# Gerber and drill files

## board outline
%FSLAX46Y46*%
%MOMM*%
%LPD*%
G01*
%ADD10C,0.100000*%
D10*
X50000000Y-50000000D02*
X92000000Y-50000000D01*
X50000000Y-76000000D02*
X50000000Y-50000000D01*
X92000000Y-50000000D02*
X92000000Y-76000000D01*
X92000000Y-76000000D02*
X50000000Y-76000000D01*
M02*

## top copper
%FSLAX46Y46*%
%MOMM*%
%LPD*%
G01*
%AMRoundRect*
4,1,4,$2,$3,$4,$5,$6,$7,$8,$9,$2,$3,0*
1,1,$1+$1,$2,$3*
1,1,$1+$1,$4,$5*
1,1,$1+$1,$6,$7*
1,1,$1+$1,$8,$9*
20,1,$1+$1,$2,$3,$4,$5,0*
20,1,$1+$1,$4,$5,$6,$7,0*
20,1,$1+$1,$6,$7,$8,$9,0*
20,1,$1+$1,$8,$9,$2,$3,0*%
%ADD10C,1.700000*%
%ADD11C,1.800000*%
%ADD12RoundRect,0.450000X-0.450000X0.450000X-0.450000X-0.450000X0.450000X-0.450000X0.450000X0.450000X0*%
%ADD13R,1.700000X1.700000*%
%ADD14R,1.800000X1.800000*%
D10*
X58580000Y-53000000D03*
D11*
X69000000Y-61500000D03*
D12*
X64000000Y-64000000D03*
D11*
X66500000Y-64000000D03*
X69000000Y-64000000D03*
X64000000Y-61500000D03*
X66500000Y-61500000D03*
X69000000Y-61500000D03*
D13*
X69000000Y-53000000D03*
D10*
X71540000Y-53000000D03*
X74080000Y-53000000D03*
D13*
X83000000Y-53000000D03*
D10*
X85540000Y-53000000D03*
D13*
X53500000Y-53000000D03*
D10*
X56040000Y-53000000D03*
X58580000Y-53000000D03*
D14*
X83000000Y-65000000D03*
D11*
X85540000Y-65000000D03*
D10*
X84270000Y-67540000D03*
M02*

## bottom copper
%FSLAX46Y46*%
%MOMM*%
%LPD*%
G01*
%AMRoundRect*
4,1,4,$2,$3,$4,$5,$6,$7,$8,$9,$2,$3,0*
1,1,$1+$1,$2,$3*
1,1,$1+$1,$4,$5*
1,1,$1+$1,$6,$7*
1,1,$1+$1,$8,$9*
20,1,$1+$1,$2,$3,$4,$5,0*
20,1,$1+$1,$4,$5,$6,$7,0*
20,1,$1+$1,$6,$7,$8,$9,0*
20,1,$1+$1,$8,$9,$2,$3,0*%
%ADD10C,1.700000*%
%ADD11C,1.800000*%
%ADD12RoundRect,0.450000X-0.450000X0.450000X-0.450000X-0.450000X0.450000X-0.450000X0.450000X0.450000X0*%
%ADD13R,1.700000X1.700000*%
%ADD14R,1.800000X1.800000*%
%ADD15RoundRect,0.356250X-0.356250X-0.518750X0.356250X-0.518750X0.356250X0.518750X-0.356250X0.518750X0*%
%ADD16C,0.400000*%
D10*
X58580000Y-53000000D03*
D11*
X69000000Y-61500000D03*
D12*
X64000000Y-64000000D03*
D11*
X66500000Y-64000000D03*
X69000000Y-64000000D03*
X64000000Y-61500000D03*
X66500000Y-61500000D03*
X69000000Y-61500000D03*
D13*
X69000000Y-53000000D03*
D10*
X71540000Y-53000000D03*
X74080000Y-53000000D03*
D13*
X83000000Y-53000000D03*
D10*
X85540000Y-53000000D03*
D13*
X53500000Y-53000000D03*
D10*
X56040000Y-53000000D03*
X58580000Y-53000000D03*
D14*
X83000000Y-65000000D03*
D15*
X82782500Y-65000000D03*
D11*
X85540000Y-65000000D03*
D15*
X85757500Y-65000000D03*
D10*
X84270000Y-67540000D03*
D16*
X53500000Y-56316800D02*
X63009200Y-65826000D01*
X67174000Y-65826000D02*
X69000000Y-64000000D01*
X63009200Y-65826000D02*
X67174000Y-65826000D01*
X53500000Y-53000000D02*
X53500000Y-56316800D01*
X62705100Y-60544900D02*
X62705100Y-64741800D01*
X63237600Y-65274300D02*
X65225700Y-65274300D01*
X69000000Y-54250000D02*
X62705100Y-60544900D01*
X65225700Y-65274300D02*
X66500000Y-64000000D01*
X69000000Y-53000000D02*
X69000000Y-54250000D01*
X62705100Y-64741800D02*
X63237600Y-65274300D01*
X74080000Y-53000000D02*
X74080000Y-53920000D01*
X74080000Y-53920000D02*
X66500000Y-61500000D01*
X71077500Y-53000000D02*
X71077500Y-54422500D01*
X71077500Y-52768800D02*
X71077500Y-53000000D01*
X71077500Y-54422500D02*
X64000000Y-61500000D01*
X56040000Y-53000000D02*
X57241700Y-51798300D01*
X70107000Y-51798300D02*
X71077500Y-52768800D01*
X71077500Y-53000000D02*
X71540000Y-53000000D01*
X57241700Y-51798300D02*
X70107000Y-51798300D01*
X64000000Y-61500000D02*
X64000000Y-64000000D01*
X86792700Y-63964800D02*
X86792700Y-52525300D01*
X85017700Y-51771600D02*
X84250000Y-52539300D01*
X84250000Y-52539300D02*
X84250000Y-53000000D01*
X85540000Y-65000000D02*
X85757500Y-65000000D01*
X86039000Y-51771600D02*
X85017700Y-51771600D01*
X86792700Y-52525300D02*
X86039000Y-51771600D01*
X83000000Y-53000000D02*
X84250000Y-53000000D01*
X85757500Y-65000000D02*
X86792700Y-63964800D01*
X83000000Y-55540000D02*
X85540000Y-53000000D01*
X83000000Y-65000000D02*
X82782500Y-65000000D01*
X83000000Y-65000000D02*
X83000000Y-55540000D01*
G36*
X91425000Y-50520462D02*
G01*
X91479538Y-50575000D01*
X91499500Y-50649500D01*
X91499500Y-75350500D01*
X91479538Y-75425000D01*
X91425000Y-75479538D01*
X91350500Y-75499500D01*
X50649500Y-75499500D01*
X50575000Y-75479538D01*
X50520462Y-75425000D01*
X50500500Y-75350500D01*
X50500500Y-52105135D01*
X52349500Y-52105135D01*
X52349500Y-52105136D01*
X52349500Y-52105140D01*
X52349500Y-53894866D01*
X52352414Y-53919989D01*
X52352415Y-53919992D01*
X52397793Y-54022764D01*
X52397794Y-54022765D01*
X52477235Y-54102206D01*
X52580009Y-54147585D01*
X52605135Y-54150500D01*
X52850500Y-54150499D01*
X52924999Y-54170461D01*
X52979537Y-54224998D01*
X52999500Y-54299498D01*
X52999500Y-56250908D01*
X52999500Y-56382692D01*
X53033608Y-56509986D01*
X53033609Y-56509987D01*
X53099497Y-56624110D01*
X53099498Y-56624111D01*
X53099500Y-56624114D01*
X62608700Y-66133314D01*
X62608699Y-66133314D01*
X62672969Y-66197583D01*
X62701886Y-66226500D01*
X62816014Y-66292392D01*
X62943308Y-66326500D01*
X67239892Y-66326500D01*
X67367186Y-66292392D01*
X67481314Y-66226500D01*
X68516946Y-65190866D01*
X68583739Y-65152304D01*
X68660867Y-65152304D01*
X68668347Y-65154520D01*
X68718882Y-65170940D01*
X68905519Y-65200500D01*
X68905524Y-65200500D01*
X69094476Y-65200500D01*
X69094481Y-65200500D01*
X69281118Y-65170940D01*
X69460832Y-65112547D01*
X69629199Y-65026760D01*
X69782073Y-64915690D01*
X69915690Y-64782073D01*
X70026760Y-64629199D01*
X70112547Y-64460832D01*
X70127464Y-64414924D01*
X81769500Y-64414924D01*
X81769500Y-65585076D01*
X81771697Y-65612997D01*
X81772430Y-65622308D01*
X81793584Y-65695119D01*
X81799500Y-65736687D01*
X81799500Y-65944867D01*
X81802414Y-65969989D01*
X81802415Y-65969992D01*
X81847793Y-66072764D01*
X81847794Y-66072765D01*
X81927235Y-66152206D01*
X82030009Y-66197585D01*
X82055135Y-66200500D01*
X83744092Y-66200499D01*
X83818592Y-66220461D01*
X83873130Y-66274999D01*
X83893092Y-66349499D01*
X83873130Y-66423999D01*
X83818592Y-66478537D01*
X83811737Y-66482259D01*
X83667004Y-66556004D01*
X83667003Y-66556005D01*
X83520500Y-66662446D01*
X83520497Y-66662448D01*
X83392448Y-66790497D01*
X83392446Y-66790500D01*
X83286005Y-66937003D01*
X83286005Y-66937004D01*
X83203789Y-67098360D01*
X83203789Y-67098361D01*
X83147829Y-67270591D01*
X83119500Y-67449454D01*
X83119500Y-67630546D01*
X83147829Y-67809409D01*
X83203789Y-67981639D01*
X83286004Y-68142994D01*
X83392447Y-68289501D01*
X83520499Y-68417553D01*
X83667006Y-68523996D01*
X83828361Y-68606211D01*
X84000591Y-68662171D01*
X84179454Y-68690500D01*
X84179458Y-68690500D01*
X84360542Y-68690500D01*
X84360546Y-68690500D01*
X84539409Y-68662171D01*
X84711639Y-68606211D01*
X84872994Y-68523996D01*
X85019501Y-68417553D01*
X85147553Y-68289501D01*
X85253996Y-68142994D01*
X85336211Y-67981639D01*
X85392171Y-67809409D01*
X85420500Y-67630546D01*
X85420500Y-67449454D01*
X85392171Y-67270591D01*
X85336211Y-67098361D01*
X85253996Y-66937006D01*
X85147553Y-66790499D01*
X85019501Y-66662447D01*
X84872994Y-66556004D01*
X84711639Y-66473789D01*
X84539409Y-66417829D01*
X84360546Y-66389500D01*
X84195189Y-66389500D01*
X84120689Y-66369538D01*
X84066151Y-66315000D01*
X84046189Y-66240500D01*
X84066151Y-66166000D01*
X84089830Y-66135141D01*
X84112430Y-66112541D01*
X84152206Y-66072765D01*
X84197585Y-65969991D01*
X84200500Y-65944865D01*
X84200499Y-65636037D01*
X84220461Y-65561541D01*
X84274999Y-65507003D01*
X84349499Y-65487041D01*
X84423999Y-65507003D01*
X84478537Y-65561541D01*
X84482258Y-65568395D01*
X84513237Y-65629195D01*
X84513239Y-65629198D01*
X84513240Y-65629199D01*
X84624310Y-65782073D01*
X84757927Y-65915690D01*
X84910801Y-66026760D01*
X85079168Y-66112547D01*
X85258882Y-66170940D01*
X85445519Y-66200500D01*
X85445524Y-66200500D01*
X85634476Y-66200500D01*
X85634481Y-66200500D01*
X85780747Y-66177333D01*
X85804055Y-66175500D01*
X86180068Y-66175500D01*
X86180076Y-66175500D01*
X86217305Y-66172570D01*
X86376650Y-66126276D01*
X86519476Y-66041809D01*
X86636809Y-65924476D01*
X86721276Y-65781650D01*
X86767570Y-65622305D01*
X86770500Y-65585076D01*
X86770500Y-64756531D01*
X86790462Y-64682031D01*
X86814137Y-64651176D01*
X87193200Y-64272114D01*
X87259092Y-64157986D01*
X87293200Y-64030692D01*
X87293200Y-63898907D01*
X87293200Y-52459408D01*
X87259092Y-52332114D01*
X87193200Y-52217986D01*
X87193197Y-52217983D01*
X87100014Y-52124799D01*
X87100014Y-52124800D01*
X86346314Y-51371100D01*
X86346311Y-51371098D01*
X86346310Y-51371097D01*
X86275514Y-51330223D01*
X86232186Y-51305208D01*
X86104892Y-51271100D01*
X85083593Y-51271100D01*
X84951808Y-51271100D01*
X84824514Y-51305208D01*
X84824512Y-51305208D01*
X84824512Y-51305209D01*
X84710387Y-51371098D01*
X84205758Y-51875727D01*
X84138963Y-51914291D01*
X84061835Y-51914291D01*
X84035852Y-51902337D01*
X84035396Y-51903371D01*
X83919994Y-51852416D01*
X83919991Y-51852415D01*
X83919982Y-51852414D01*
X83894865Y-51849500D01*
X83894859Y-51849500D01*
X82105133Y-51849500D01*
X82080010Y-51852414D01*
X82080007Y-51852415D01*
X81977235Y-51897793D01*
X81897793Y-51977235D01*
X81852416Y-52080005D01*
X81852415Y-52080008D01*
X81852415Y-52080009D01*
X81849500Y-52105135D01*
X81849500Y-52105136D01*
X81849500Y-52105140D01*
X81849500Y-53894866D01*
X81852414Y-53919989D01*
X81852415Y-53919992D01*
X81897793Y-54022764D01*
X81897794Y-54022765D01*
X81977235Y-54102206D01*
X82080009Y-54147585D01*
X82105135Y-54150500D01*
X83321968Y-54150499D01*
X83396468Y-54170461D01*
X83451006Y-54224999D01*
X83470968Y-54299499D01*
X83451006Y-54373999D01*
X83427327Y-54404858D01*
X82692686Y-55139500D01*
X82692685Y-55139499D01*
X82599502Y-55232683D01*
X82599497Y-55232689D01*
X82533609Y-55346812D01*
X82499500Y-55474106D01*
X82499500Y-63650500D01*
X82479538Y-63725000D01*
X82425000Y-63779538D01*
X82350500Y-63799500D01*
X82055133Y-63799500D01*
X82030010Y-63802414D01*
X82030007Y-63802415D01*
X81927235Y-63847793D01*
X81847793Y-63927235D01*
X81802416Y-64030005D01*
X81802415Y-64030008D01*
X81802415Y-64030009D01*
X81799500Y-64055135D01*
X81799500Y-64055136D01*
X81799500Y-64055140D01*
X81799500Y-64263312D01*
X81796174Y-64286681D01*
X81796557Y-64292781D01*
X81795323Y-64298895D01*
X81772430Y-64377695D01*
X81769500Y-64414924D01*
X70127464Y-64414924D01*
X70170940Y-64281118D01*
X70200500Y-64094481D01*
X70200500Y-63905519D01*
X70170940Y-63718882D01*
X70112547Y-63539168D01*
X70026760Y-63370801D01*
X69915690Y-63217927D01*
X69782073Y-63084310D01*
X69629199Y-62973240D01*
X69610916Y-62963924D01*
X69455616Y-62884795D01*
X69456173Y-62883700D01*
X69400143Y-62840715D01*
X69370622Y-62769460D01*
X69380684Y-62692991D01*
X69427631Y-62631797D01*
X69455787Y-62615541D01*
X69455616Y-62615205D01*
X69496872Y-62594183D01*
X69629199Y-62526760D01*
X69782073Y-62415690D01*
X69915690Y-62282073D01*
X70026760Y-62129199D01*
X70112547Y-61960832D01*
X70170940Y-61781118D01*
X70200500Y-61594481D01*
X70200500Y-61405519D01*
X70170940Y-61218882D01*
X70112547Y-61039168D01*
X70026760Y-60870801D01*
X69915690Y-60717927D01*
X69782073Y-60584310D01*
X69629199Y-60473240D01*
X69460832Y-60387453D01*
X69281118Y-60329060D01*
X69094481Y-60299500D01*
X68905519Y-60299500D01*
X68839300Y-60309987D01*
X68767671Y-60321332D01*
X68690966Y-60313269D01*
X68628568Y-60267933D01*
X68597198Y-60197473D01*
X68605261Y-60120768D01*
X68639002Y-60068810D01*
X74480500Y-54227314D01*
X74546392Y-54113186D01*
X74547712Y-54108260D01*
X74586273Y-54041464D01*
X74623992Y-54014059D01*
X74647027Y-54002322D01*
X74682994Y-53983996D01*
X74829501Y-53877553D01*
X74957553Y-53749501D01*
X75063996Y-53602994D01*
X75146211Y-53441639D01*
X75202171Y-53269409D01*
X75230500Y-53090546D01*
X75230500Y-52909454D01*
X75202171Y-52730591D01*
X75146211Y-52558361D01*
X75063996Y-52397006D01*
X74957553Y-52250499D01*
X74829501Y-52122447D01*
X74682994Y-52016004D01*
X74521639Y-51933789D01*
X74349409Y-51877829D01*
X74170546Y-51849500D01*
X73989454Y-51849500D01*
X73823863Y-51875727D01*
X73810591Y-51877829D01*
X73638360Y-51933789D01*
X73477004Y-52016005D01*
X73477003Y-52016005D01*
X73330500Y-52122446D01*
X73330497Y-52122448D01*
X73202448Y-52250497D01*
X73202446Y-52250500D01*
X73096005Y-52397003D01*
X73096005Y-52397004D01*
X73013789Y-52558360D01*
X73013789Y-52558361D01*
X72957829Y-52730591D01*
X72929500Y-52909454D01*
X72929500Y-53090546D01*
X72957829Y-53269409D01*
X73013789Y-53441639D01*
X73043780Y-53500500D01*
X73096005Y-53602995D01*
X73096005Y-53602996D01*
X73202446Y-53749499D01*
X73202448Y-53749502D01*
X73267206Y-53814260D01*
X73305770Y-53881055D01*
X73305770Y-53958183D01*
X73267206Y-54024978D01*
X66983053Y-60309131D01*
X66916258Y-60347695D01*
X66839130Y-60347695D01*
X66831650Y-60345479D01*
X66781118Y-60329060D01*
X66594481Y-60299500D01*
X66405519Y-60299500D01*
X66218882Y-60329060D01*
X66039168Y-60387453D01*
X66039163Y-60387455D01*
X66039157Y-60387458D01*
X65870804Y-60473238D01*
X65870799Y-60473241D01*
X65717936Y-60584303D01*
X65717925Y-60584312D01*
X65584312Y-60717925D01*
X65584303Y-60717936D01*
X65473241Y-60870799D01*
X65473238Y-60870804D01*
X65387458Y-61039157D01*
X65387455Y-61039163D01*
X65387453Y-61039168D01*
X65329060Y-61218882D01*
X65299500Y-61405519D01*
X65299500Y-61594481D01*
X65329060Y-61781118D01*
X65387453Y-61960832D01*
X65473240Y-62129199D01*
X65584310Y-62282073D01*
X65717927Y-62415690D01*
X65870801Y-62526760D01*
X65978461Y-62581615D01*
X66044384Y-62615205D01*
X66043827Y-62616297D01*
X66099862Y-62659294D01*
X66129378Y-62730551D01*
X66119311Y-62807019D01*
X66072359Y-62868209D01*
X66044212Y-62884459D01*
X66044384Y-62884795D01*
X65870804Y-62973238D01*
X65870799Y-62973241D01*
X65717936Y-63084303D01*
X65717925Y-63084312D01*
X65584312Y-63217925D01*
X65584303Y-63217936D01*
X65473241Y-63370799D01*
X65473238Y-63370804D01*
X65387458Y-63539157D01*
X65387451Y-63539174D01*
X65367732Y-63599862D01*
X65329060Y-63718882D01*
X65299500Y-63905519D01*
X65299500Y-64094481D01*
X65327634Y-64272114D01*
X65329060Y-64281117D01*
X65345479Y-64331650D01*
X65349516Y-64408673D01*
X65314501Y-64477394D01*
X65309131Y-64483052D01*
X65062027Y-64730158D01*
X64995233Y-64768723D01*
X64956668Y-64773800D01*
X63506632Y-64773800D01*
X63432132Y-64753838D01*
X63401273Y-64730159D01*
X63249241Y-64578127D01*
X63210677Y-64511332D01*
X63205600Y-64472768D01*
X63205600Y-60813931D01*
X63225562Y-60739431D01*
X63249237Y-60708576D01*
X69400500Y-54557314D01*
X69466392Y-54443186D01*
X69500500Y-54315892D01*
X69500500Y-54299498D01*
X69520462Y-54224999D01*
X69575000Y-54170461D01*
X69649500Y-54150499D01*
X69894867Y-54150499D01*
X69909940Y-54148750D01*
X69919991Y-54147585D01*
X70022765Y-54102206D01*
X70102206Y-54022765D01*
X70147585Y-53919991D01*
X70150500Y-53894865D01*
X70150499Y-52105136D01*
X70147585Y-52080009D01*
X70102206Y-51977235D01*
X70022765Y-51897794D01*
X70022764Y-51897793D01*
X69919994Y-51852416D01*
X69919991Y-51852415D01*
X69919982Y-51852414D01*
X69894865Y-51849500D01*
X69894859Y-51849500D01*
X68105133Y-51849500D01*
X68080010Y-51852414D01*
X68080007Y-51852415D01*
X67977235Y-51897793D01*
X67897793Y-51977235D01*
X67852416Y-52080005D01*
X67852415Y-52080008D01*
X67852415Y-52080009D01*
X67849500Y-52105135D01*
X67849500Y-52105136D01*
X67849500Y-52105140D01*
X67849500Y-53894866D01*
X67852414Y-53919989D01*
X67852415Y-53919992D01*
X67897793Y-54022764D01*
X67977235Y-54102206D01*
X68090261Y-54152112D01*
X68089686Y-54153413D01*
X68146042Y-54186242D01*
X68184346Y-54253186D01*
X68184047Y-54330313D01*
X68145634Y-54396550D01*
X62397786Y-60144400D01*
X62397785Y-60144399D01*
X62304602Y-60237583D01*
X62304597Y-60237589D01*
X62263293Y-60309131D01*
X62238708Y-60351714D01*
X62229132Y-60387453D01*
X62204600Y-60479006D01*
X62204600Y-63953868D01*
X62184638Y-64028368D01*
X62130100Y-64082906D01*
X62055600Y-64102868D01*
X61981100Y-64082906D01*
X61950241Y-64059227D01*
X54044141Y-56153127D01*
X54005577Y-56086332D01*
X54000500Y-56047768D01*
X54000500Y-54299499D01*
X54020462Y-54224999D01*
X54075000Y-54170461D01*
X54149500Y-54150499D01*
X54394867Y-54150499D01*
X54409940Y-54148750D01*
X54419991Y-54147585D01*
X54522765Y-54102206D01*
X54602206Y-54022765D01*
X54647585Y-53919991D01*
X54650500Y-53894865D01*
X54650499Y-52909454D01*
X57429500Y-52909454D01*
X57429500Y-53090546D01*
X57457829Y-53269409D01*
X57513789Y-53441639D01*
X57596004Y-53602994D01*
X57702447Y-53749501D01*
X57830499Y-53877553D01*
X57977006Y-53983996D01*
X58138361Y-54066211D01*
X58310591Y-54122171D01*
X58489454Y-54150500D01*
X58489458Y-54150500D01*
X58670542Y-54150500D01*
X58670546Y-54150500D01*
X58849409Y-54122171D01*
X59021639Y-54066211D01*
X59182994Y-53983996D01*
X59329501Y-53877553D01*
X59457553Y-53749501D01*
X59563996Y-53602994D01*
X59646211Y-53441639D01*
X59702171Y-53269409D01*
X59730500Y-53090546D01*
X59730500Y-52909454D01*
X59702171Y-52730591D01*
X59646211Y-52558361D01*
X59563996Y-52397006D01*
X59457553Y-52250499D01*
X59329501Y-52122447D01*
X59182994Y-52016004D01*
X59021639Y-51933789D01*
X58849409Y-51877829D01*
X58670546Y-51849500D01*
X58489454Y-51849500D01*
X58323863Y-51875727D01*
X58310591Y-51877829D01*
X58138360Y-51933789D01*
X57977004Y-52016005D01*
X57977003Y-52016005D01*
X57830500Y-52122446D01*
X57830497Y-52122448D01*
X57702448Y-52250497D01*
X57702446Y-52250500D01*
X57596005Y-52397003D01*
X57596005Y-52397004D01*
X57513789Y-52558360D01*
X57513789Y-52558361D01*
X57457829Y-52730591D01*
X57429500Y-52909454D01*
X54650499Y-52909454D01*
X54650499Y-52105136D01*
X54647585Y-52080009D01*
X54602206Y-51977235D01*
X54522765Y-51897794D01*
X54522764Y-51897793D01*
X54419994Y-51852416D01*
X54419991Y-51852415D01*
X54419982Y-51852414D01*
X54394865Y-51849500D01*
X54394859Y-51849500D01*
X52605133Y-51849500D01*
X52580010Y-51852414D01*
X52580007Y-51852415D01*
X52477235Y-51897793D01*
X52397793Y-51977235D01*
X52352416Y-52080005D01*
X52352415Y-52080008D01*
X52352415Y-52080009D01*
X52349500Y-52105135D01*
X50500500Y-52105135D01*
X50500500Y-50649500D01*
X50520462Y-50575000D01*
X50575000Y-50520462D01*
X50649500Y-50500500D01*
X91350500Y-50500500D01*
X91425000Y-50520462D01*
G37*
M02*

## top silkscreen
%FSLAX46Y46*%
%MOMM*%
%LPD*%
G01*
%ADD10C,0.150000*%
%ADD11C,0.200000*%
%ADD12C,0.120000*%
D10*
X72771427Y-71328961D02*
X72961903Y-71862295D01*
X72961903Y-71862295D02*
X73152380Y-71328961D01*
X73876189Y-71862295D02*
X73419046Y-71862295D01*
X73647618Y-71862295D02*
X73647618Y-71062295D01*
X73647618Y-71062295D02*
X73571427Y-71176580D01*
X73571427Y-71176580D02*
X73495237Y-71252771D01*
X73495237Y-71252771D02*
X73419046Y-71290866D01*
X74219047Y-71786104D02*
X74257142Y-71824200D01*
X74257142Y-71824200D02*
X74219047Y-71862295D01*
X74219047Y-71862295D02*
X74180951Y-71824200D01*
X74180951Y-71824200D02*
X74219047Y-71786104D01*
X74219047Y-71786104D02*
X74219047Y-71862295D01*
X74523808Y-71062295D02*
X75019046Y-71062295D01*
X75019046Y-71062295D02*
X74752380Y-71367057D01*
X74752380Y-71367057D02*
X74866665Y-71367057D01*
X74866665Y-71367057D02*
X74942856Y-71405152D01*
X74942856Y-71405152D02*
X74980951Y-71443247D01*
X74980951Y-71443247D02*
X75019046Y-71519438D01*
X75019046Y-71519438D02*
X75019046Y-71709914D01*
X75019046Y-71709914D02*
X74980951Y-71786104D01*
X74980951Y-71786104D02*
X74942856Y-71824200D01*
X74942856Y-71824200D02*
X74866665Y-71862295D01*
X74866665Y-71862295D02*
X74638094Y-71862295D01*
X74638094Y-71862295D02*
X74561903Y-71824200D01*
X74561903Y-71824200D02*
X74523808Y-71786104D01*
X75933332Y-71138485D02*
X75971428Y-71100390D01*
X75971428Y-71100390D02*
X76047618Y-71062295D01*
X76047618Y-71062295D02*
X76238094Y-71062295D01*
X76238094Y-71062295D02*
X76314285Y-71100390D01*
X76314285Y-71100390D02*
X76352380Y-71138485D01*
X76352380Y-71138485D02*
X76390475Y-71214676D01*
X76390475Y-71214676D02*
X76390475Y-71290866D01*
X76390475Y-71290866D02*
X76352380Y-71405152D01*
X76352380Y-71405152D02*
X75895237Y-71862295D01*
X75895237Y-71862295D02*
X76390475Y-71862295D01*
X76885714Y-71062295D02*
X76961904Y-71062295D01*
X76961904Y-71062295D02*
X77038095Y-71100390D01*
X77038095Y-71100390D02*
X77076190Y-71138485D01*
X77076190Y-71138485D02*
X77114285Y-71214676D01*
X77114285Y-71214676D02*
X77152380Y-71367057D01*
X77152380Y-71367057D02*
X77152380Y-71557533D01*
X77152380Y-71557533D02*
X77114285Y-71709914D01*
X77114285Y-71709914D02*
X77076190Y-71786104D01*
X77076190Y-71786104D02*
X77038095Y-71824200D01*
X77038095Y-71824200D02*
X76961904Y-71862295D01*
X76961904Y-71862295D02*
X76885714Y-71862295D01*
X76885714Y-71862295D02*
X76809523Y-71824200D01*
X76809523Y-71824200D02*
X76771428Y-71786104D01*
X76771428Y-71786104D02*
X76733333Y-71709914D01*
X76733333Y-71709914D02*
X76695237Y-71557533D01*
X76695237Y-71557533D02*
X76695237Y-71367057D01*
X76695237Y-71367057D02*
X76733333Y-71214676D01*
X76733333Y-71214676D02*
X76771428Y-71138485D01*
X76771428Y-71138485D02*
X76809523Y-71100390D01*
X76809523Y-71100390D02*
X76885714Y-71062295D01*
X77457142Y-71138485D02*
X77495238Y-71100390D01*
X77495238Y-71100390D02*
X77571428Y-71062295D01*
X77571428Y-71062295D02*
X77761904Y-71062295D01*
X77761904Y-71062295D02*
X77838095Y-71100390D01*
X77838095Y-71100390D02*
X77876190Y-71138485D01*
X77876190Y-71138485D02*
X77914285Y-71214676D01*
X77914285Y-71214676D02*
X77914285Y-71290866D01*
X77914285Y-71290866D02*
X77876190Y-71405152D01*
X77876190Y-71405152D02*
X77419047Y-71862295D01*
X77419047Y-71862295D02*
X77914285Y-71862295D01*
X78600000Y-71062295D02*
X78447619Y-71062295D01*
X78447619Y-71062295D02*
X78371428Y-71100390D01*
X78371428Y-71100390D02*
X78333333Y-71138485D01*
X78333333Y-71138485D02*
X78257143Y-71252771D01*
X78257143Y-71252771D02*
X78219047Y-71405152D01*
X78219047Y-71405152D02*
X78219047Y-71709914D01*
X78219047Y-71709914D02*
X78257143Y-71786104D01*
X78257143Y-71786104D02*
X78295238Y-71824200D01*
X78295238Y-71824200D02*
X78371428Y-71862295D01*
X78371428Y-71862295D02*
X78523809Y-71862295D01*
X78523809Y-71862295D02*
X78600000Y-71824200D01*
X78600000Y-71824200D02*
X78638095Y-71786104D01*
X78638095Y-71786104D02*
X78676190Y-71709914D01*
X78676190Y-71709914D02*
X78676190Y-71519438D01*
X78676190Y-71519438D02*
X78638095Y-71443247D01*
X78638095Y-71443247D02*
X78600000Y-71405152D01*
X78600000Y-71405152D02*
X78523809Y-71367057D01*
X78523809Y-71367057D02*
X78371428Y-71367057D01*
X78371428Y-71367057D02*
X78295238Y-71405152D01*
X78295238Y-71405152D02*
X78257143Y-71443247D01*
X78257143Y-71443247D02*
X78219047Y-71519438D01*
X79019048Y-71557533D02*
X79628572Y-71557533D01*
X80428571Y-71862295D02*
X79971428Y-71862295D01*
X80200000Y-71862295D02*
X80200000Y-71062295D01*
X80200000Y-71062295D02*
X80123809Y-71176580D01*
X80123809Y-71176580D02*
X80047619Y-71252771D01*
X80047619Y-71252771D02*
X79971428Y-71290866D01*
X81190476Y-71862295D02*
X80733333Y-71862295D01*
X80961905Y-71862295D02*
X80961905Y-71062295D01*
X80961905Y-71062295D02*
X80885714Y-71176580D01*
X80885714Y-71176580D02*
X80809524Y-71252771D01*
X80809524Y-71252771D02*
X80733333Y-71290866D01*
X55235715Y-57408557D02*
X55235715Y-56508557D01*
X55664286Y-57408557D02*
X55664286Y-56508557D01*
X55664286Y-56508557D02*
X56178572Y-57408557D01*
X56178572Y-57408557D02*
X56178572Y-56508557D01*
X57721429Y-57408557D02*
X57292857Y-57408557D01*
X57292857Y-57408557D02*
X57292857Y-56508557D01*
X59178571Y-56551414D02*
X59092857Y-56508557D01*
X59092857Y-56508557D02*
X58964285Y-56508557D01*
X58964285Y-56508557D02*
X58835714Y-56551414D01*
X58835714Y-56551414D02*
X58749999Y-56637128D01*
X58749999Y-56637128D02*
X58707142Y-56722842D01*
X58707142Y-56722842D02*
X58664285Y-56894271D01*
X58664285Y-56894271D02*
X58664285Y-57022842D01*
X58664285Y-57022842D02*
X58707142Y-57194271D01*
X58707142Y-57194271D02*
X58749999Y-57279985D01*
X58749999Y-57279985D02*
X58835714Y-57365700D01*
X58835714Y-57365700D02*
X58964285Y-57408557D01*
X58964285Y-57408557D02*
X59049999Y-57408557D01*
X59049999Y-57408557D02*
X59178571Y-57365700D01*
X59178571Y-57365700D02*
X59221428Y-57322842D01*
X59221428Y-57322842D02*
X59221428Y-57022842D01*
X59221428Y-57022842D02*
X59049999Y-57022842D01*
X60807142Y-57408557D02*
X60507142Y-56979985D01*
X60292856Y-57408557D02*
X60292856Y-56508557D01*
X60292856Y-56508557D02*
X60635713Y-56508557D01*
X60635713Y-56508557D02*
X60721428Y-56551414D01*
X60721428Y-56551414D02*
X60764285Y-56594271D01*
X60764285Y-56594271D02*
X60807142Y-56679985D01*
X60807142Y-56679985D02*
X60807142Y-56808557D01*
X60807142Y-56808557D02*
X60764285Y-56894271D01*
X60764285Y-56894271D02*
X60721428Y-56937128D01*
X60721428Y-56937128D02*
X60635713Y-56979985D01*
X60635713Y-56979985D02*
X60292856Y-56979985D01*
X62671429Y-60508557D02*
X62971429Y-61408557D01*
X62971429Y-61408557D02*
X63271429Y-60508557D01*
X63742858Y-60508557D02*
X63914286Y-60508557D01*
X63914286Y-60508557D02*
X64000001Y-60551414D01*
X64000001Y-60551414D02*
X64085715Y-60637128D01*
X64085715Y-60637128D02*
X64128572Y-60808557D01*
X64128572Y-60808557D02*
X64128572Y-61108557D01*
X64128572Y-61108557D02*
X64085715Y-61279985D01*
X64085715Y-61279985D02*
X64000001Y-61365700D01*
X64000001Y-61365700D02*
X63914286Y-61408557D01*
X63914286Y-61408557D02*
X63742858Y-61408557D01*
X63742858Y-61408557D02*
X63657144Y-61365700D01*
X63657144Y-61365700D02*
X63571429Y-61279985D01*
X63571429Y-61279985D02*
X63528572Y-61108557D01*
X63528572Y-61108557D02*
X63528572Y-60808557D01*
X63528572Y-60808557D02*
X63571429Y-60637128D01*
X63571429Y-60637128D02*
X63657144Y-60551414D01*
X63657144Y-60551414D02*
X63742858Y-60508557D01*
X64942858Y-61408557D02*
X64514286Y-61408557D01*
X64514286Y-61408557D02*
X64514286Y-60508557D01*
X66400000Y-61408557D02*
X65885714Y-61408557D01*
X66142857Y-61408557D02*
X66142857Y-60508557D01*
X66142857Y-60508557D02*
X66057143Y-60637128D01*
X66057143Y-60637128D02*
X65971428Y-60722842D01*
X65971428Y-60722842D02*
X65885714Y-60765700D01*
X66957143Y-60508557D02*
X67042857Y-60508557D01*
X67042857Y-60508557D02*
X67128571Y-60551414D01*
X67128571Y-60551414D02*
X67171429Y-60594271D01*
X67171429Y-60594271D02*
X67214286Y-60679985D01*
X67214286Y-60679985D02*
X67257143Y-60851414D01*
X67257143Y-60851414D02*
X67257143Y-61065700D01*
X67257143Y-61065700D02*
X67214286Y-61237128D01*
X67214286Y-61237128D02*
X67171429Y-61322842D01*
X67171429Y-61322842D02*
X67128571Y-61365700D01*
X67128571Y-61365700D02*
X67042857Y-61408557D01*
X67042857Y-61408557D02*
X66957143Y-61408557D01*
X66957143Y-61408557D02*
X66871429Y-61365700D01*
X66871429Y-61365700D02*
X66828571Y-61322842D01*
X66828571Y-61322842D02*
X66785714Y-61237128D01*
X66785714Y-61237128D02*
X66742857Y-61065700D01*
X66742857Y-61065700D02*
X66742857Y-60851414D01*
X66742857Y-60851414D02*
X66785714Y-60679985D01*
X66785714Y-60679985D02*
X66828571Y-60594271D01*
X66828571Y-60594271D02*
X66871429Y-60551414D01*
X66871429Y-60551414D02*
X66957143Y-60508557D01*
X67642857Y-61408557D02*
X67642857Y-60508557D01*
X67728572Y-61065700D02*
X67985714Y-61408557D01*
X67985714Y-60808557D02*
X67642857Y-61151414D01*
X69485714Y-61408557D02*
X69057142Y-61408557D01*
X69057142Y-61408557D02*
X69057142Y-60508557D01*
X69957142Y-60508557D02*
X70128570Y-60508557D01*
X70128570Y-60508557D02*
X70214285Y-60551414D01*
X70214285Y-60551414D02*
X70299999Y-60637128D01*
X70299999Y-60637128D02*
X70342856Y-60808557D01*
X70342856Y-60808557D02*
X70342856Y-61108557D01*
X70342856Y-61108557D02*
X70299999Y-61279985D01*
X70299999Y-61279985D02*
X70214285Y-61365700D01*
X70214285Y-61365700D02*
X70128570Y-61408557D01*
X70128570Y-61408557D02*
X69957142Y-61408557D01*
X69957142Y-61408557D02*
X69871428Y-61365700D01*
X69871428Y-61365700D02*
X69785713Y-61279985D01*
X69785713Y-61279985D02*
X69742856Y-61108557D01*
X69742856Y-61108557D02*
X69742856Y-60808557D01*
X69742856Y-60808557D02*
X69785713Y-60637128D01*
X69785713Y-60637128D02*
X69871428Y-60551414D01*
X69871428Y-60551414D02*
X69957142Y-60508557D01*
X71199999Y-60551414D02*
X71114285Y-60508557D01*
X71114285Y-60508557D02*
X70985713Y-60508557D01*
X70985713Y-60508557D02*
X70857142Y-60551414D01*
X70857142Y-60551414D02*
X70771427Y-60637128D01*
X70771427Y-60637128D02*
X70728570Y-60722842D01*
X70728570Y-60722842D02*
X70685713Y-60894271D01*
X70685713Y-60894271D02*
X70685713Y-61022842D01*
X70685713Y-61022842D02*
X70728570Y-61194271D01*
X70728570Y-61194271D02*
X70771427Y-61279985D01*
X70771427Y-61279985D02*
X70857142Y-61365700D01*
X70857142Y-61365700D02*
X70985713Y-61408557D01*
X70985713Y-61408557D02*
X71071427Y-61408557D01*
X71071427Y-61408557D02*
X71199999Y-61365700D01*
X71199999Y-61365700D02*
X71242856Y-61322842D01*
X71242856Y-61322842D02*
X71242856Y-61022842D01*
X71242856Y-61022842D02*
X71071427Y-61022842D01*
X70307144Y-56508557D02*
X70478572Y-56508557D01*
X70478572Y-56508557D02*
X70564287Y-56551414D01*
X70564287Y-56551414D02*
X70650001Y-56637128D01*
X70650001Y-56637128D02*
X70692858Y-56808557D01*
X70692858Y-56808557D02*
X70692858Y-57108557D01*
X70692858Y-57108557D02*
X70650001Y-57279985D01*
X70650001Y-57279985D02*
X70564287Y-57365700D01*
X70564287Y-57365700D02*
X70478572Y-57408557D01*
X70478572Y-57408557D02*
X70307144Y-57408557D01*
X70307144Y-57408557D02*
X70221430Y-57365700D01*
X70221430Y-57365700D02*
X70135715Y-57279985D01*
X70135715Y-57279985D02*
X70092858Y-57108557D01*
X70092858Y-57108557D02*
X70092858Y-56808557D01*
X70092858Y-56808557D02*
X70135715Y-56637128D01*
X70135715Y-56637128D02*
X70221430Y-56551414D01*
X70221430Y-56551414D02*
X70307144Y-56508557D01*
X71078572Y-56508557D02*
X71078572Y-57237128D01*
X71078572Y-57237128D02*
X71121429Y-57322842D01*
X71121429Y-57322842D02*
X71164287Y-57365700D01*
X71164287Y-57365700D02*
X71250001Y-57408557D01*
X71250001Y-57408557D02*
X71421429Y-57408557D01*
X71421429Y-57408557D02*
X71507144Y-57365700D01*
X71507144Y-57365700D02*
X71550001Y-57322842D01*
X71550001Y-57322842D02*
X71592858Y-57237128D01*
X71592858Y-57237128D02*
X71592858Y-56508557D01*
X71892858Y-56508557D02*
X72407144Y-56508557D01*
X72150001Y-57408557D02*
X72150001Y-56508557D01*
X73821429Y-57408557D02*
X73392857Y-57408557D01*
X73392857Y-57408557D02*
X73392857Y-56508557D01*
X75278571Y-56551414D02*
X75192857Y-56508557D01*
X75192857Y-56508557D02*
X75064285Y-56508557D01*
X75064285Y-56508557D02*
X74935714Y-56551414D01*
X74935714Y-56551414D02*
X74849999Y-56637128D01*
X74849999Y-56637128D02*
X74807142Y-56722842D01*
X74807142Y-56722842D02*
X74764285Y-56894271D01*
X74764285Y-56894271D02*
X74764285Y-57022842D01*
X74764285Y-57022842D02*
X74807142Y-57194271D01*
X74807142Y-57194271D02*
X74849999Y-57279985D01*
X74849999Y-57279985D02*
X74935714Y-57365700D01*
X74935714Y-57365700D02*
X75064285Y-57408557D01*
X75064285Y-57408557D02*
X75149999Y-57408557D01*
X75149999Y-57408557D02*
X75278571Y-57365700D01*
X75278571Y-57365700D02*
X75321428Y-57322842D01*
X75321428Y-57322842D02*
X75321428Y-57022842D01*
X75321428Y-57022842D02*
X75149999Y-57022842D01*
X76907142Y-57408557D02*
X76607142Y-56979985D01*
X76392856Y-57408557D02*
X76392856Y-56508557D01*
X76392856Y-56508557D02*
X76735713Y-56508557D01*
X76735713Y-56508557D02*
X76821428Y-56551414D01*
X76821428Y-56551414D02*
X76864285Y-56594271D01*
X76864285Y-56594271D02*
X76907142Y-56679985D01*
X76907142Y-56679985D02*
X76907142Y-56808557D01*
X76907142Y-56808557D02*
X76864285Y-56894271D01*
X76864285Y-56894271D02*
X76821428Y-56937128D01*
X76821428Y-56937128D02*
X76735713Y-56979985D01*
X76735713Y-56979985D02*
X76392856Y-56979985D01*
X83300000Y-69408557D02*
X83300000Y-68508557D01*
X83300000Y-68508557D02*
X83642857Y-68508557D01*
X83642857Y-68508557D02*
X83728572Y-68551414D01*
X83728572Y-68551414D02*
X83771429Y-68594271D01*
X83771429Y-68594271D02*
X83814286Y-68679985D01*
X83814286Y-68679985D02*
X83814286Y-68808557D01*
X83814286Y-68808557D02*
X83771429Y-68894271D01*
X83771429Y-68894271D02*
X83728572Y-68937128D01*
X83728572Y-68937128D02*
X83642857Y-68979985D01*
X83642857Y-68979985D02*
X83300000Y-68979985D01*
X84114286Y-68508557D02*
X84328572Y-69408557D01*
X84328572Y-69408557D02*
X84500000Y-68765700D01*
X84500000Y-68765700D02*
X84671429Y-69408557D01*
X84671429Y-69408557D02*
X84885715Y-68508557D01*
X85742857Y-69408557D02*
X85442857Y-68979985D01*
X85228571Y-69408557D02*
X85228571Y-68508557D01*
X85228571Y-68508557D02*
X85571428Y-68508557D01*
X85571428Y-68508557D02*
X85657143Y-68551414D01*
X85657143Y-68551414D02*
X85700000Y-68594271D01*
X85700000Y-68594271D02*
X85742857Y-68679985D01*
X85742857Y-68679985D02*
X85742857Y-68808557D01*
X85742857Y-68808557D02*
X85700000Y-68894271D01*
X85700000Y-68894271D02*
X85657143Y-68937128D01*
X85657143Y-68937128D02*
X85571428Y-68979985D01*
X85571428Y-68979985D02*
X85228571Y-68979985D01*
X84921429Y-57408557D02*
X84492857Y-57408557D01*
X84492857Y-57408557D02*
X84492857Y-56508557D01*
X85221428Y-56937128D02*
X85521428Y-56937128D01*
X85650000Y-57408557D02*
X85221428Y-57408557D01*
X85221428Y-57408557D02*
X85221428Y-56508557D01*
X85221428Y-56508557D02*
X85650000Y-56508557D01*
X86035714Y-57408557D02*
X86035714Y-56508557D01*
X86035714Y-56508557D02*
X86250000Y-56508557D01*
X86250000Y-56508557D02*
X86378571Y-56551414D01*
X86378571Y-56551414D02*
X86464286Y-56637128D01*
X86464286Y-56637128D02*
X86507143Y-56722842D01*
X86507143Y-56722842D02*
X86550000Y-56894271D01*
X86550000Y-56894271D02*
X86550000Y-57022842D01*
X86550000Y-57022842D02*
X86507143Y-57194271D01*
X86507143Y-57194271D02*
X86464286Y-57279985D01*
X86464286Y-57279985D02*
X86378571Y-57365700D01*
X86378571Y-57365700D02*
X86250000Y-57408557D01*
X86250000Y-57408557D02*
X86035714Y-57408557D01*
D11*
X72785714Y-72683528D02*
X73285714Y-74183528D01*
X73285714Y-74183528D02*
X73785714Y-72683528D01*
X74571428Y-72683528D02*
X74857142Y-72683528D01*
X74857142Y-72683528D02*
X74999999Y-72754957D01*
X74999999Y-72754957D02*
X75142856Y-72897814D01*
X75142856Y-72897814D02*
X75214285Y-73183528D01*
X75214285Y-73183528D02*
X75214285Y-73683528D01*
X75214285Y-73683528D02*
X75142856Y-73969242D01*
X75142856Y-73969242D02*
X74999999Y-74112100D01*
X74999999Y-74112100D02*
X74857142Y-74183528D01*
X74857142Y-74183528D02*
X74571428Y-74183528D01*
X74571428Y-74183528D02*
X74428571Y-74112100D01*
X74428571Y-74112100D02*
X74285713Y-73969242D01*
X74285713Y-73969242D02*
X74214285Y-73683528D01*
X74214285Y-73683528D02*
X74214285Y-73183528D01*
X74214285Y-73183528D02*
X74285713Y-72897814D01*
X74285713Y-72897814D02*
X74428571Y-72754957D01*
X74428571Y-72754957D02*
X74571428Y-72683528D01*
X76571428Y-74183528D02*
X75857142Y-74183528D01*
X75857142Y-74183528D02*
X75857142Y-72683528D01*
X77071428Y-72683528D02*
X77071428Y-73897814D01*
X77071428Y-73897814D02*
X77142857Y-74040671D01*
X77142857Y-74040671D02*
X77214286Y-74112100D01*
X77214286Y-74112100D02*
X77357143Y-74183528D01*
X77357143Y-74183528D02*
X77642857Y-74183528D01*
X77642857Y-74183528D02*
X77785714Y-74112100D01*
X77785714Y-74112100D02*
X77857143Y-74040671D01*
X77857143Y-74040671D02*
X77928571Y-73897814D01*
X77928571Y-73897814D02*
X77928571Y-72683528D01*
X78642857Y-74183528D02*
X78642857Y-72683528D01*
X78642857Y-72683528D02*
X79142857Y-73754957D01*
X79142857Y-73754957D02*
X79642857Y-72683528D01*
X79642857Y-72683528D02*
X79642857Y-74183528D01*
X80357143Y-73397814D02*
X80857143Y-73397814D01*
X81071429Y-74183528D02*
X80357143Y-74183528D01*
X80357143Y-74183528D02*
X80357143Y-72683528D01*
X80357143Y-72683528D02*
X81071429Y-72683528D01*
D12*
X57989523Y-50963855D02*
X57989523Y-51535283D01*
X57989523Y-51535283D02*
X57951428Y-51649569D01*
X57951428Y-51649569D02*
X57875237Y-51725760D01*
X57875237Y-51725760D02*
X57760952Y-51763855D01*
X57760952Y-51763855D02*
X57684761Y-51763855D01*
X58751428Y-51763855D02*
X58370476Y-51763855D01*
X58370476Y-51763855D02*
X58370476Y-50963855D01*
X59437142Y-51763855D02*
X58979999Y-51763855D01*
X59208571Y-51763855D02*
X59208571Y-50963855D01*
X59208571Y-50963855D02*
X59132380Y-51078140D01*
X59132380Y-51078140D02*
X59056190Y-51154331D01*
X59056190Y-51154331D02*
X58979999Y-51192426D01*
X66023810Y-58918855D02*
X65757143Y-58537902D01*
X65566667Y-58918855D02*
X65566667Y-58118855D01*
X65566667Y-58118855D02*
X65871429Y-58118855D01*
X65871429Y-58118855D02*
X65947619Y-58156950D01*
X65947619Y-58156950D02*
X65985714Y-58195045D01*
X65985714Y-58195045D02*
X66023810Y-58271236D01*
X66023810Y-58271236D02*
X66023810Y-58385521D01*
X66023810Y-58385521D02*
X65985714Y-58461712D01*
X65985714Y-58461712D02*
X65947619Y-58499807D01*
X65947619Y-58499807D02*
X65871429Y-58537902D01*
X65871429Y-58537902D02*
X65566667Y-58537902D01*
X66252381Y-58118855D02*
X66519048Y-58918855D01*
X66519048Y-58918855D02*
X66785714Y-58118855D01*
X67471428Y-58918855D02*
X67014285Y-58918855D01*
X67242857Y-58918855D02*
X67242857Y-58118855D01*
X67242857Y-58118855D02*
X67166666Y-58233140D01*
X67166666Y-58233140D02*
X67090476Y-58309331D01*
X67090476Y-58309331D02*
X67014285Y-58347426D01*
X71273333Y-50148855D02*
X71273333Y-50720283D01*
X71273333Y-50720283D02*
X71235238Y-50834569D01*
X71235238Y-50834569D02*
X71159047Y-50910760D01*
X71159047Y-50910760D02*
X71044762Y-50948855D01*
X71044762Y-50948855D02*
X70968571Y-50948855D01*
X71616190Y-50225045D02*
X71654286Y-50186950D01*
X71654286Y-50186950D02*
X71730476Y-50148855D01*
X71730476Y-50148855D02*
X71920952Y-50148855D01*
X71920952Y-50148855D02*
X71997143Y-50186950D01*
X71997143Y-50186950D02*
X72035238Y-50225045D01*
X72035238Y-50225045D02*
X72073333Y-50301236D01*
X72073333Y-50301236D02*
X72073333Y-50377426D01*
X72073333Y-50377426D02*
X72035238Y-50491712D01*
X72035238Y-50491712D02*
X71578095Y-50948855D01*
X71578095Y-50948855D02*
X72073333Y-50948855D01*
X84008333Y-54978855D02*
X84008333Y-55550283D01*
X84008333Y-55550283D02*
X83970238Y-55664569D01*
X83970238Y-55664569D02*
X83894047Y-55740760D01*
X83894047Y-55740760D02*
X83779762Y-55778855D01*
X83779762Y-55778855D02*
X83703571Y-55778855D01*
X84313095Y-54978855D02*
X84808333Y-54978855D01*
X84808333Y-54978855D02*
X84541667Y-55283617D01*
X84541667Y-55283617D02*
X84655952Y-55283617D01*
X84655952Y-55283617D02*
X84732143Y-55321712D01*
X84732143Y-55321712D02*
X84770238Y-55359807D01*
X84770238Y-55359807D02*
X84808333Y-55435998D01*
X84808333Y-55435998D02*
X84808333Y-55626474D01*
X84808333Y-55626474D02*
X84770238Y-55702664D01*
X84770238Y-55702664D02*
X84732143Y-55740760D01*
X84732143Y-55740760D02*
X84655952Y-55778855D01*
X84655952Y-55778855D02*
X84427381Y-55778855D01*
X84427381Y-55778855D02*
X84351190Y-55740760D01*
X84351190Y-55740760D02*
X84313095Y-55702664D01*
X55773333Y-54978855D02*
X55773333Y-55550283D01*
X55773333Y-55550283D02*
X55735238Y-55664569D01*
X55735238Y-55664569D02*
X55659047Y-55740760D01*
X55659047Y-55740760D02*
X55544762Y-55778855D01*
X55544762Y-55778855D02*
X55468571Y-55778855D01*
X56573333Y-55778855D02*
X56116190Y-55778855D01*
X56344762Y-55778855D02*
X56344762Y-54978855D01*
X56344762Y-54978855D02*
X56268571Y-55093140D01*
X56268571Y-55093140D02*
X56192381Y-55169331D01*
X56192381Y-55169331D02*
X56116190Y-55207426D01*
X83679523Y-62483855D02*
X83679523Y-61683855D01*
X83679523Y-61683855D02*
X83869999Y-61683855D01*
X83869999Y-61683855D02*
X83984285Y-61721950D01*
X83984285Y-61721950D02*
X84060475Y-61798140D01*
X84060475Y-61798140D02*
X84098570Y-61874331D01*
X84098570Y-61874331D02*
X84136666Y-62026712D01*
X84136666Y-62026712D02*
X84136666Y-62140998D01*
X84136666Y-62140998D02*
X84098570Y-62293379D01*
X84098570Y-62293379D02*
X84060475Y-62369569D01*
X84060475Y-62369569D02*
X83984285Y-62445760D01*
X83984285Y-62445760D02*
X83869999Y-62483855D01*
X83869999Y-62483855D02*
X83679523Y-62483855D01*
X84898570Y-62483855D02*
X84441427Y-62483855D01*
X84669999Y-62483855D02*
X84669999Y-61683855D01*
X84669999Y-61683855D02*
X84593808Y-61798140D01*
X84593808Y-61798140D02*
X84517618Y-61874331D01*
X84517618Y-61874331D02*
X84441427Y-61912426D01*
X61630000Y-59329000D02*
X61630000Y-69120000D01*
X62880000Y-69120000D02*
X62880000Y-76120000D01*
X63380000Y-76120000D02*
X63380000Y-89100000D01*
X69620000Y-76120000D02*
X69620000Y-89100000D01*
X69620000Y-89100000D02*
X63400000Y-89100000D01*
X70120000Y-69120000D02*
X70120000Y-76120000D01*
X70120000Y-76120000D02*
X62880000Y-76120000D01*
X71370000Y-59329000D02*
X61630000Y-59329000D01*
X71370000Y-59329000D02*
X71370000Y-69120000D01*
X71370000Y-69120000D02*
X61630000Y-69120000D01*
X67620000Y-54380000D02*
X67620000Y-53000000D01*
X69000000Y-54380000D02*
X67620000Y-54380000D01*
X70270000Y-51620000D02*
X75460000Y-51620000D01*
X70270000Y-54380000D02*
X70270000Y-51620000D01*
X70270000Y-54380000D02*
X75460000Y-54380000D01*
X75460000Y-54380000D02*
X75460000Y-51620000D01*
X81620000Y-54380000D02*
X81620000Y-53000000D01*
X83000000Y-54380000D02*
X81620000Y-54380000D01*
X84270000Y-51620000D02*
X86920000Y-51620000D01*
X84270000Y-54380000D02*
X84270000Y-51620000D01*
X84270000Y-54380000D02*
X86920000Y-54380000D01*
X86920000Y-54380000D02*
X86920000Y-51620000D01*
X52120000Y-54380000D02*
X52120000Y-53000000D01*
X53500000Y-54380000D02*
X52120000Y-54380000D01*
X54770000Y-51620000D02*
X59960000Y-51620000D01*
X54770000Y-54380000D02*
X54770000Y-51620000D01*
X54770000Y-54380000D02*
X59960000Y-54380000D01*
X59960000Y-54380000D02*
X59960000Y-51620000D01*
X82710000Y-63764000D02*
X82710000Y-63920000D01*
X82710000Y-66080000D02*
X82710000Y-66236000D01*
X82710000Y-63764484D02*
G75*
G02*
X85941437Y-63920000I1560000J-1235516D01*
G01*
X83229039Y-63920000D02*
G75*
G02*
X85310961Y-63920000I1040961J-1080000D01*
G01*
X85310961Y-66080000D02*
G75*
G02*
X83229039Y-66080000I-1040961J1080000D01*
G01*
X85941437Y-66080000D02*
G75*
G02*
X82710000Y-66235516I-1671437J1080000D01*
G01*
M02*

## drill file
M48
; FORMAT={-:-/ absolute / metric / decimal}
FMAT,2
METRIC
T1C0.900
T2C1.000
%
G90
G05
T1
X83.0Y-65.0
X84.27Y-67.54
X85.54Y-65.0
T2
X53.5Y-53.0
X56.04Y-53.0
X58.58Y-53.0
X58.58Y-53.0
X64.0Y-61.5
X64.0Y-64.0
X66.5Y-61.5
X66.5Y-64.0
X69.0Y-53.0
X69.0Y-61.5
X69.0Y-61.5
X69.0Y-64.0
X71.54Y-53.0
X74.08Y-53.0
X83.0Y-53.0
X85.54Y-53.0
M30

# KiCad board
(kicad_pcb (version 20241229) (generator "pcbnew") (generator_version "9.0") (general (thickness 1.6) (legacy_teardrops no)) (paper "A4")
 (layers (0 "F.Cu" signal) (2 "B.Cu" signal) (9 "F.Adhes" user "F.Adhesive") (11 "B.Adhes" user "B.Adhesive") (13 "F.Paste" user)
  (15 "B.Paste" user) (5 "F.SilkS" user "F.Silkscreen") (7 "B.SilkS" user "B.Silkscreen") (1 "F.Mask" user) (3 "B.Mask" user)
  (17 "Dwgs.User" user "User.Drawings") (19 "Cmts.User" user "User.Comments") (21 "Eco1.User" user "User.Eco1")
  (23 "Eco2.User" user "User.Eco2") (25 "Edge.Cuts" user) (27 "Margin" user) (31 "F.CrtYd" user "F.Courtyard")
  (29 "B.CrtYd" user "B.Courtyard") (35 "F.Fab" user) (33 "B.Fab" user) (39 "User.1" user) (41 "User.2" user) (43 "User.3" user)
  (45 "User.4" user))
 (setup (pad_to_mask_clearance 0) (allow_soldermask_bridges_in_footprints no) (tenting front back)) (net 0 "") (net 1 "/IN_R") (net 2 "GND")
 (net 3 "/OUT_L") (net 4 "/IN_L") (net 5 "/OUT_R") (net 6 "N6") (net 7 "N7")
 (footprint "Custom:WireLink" (layer "F.Cu") (at 58.58 53)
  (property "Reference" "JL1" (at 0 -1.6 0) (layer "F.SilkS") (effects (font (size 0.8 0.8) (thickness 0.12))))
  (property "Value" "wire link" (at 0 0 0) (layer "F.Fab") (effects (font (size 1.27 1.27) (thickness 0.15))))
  (pad "1" thru_hole circle (at 0 0) (size 1.7 1.7) (drill 1) (layers "*.Cu" "*.Mask") (remove_unused_layers no) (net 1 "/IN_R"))
  (pad "2" thru_hole circle (at 10.42 8.5) (size 1.8 1.8) (drill 1) (layers "*.Cu" "*.Mask") (remove_unused_layers no) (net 1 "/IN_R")))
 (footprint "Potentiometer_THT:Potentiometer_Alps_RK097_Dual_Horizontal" (layer "F.Cu") (at 64 64 90)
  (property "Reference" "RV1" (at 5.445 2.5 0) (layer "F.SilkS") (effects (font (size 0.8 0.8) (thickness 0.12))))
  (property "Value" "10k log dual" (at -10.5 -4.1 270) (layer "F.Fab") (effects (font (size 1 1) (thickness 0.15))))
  (fp_line (start 4.671 -2.37) (end -5.12 -2.37) (stroke (width 0.12) (type solid)) (layer "F.SilkS"))
  (fp_line (start -5.12 -1.12) (end -12.12 -1.12) (stroke (width 0.12) (type solid)) (layer "F.SilkS"))
  (fp_line (start -12.12 -0.62) (end -25.1 -0.62) (stroke (width 0.12) (type solid)) (layer "F.SilkS"))
  (fp_line (start -12.12 5.62) (end -25.1 5.62) (stroke (width 0.12) (type solid)) (layer "F.SilkS"))
  (fp_line (start -25.1 5.62) (end -25.1 -0.6) (stroke (width 0.12) (type solid)) (layer "F.SilkS"))
  (fp_line (start -5.12 6.12) (end -12.12 6.12) (stroke (width 0.12) (type solid)) (layer "F.SilkS"))
  (fp_line (start -12.12 6.12) (end -12.12 -1.12) (stroke (width 0.12) (type solid)) (layer "F.SilkS"))
  (fp_line (start 4.671 7.37) (end 4.671 -2.37) (stroke (width 0.12) (type solid)) (layer "F.SilkS"))
  (fp_line (start 4.671 7.37) (end -5.12 7.37) (stroke (width 0.12) (type solid)) (layer "F.SilkS"))
  (fp_line (start -5.12 7.37) (end -5.12 -2.37) (stroke (width 0.12) (type solid)) (layer "F.SilkS"))
  (pad "1" thru_hole roundrect (at 0 0 270) (size 1.8 1.8) (drill 1) (layers "*.Cu" "*.Mask") (remove_unused_layers no)
   (roundrect_rratio 0.25) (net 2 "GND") (zone_connect 2))
  (pad "2" thru_hole circle (at 0 2.5 270) (size 1.8 1.8) (drill 1) (layers "*.Cu" "*.Mask") (remove_unused_layers no) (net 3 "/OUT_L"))
  (pad "3" thru_hole circle (at 0 5 270) (size 1.8 1.8) (drill 1) (layers "*.Cu" "*.Mask") (remove_unused_layers no) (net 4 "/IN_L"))
  (pad "4" thru_hole circle (at 2.5 0 270) (size 1.8 1.8) (drill 1) (layers "*.Cu" "*.Mask") (remove_unused_layers no) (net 2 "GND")
   (zone_connect 2))
  (pad "5" thru_hole circle (at 2.5 2.5 270) (size 1.8 1.8) (drill 1) (layers "*.Cu" "*.Mask") (remove_unused_layers no) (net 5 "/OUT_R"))
  (pad "6" thru_hole circle (at 2.5 5 270) (size 1.8 1.8) (drill 1) (layers "*.Cu" "*.Mask") (remove_unused_layers no) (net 1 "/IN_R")))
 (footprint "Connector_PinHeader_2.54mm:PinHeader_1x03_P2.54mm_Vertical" (layer "F.Cu") (at 69 53 90)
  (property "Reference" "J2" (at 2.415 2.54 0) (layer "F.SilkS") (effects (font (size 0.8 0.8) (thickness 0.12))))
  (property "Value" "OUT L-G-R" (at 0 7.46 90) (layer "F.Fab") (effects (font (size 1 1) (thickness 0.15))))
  (fp_line (start -1.38 -1.38) (end 0 -1.38) (stroke (width 0.12) (type solid)) (layer "F.SilkS"))
  (fp_line (start -1.38 0) (end -1.38 -1.38) (stroke (width 0.12) (type solid)) (layer "F.SilkS"))
  (fp_line (start 1.38 1.27) (end 1.38 6.46) (stroke (width 0.12) (type solid)) (layer "F.SilkS"))
  (fp_line (start -1.38 1.27) (end 1.38 1.27) (stroke (width 0.12) (type solid)) (layer "F.SilkS"))
  (fp_line (start -1.38 1.27) (end -1.38 6.46) (stroke (width 0.12) (type solid)) (layer "F.SilkS"))
  (fp_line (start -1.38 6.46) (end 1.38 6.46) (stroke (width 0.12) (type solid)) (layer "F.SilkS"))
  (pad "1" thru_hole rect (at 0 0 90) (size 1.7 1.7) (drill 1) (layers "*.Cu" "*.Mask") (remove_unused_layers no) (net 3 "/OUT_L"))
  (pad "2" thru_hole circle (at 0 2.54 90) (size 1.7 1.7) (drill 1) (layers "*.Cu" "*.Mask") (remove_unused_layers no) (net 2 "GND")
   (zone_connect 2))
  (pad "3" thru_hole circle (at 0 5.08 90) (size 1.7 1.7) (drill 1) (layers "*.Cu" "*.Mask") (remove_unused_layers no) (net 5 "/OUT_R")))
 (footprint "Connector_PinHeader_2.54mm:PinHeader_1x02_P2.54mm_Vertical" (layer "F.Cu") (at 83 53 90)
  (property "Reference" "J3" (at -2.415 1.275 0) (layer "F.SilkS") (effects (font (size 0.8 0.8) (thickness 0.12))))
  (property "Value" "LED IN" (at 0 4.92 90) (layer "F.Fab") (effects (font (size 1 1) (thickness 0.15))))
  (fp_line (start -1.38 -1.38) (end 0 -1.38) (stroke (width 0.12) (type solid)) (layer "F.SilkS"))
  (fp_line (start -1.38 0) (end -1.38 -1.38) (stroke (width 0.12) (type solid)) (layer "F.SilkS"))
  (fp_line (start 1.38 1.27) (end 1.38 3.92) (stroke (width 0.12) (type solid)) (layer "F.SilkS"))
  (fp_line (start -1.38 1.27) (end 1.38 1.27) (stroke (width 0.12) (type solid)) (layer "F.SilkS"))
  (fp_line (start -1.38 1.27) (end -1.38 3.92) (stroke (width 0.12) (type solid)) (layer "F.SilkS"))
  (fp_line (start -1.38 3.92) (end 1.38 3.92) (stroke (width 0.12) (type solid)) (layer "F.SilkS"))
  (pad "1" thru_hole rect (at 0 0 90) (size 1.7 1.7) (drill 1) (layers "*.Cu" "*.Mask") (remove_unused_layers no) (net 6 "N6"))
  (pad "2" thru_hole circle (at 0 2.54 90) (size 1.7 1.7) (drill 1) (layers "*.Cu" "*.Mask") (remove_unused_layers no) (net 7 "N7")))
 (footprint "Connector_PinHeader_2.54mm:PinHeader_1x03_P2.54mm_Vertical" (layer "F.Cu") (at 53.5 53 90)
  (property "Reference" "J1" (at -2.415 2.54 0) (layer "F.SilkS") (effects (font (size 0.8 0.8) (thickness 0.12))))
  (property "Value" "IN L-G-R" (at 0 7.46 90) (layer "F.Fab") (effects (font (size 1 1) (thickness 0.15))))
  (fp_line (start -1.38 -1.38) (end 0 -1.38) (stroke (width 0.12) (type solid)) (layer "F.SilkS"))
  (fp_line (start -1.38 0) (end -1.38 -1.38) (stroke (width 0.12) (type solid)) (layer "F.SilkS"))
  (fp_line (start 1.38 1.27) (end 1.38 6.46) (stroke (width 0.12) (type solid)) (layer "F.SilkS"))
  (fp_line (start -1.38 1.27) (end 1.38 1.27) (stroke (width 0.12) (type solid)) (layer "F.SilkS"))
  (fp_line (start -1.38 1.27) (end -1.38 6.46) (stroke (width 0.12) (type solid)) (layer "F.SilkS"))
  (fp_line (start -1.38 6.46) (end 1.38 6.46) (stroke (width 0.12) (type solid)) (layer "F.SilkS"))
  (pad "1" thru_hole rect (at 0 0 90) (size 1.7 1.7) (drill 1) (layers "*.Cu" "*.Mask") (remove_unused_layers no) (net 4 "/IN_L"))
  (pad "2" thru_hole circle (at 0 2.54 90) (size 1.7 1.7) (drill 1) (layers "*.Cu" "*.Mask") (remove_unused_layers no) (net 2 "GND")
   (zone_connect 2))
  (pad "3" thru_hole circle (at 0 5.08 90) (size 1.7 1.7) (drill 1) (layers "*.Cu" "*.Mask") (remove_unused_layers no) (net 1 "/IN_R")))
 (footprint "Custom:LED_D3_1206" (layer "F.Cu") (at 83 65)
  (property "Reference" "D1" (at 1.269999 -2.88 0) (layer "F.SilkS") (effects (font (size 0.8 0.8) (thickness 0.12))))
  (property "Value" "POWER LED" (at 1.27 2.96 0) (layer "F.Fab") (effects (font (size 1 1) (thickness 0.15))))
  (fp_line (start -0.29 -1.236) (end -0.29 -1.08) (stroke (width 0.12) (type solid)) (layer "F.SilkS"))
  (fp_line (start -0.29 1.08) (end -0.29 1.236) (stroke (width 0.12) (type solid)) (layer "F.SilkS"))
  (fp_arc (start -0.29 -1.235516) (mid 1.36566 -1.987699) (end 2.941437 -1.08) (stroke (width 0.12) (type solid)) (layer "F.SilkS"))
  (fp_arc (start 0.229039 -1.08) (mid 1.27 -1.5) (end 2.310961 -1.08) (stroke (width 0.12) (type solid)) (layer "F.SilkS"))
  (fp_arc (start 2.310961 1.08) (mid 1.27 1.5) (end 0.229039 1.08) (stroke (width 0.12) (type solid)) (layer "F.SilkS"))
  (fp_arc (start 2.941437 1.08) (mid 1.36566 1.987699) (end -0.29 1.235516) (stroke (width 0.12) (type solid)) (layer "F.SilkS"))
  (pad "1" thru_hole rect (at 0 0) (size 1.8 1.8) (drill 0.9) (layers "*.Cu" "*.Mask") (remove_unused_layers no) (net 7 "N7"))
  (pad "1S" smd roundrect (at -0.2175 0) (size 1.425 1.75) (layers "B.Cu" "B.Mask" "B.Paste") (roundrect_rratio 0.25) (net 7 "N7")
   (zone_connect 2) (thermal_bridge_angle 45))
  (pad "2" thru_hole circle (at 2.54 0) (size 1.8 1.8) (drill 0.9) (layers "*.Cu" "*.Mask") (remove_unused_layers no) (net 6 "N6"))
  (pad "2S" smd roundrect (at 2.7575 0) (size 1.425 1.75) (layers "B.Cu" "B.Mask" "B.Paste") (roundrect_rratio 0.25) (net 6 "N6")
   (zone_connect 2) (thermal_bridge_angle 45))
  (pad "M" thru_hole circle (at 1.27 2.54) (size 1.7 1.7) (drill 0.9) (layers "*.Cu" "*.Mask") (remove_unused_layers no)))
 (gr_line (start 50 50) (end 92 50) (stroke (width 0.1) (type default)) (layer "Edge.Cuts"))
 (gr_line (start 50 76) (end 50 50) (stroke (width 0.1) (type default)) (layer "Edge.Cuts"))
 (gr_line (start 92 50) (end 92 76) (stroke (width 0.1) (type default)) (layer "Edge.Cuts"))
 (gr_line (start 92 76) (end 50 76) (stroke (width 0.1) (type default)) (layer "Edge.Cuts"))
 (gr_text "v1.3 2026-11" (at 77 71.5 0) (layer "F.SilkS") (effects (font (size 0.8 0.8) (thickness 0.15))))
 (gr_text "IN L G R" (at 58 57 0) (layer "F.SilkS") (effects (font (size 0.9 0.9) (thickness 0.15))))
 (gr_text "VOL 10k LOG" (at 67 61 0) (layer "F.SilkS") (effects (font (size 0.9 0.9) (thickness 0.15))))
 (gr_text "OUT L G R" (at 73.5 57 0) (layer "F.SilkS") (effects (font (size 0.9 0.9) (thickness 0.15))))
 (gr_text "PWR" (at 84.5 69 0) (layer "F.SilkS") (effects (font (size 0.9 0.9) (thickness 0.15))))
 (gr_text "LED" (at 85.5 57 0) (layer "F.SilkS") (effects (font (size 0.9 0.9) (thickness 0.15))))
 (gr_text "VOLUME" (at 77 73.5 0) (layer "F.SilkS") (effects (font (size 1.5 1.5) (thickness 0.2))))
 (segment (start 53.5 56.3168) (end 63.0092 65.826) (width 0.4) (layer "B.Cu") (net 4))
 (segment (start 67.174 65.826) (end 69 64) (width 0.4) (layer "B.Cu") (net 4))
 (segment (start 63.0092 65.826) (end 67.174 65.826) (width 0.4) (layer "B.Cu") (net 4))
 (segment (start 53.5 53) (end 53.5 56.3168) (width 0.4) (layer "B.Cu") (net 4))
 (segment (start 62.7051 60.5449) (end 62.7051 64.7418) (width 0.4) (layer "B.Cu") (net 3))
 (segment (start 63.2376 65.2743) (end 65.2257 65.2743) (width 0.4) (layer "B.Cu") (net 3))
 (segment (start 69 54.25) (end 62.7051 60.5449) (width 0.4) (layer "B.Cu") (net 3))
 (segment (start 65.2257 65.2743) (end 66.5 64) (width 0.4) (layer "B.Cu") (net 3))
 (segment (start 69 53) (end 69 54.25) (width 0.4) (layer "B.Cu") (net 3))
 (segment (start 62.7051 64.7418) (end 63.2376 65.2743) (width 0.4) (layer "B.Cu") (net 3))
 (segment (start 74.08 53) (end 74.08 53.92) (width 0.4) (layer "B.Cu") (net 5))
 (segment (start 74.08 53.92) (end 66.5 61.5) (width 0.4) (layer "B.Cu") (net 5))
 (segment (start 71.0775 53) (end 71.0775 54.4225) (width 0.4) (layer "B.Cu") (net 2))
 (segment (start 71.0775 52.7688) (end 71.0775 53) (width 0.4) (layer "B.Cu") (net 2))
 (segment (start 71.0775 54.4225) (end 64 61.5) (width 0.4) (layer "B.Cu") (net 2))
 (segment (start 56.04 53) (end 57.2417 51.7983) (width 0.4) (layer "B.Cu") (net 2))
 (segment (start 70.107 51.7983) (end 71.0775 52.7688) (width 0.4) (layer "B.Cu") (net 2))
 (segment (start 71.0775 53) (end 71.54 53) (width 0.4) (layer "B.Cu") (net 2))
 (segment (start 57.2417 51.7983) (end 70.107 51.7983) (width 0.4) (layer "B.Cu") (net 2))
 (segment (start 64 61.5) (end 64 64) (width 0.4) (layer "B.Cu") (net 2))
 (segment (start 86.7927 63.9648) (end 86.7927 52.5253) (width 0.4) (layer "B.Cu") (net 6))
 (segment (start 85.0177 51.7716) (end 84.25 52.5393) (width 0.4) (layer "B.Cu") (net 6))
 (segment (start 84.25 52.5393) (end 84.25 53) (width 0.4) (layer "B.Cu") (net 6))
 (segment (start 85.54 65) (end 85.7575 65) (width 0.4) (layer "B.Cu") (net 6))
 (segment (start 86.039 51.7716) (end 85.0177 51.7716) (width 0.4) (layer "B.Cu") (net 6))
 (segment (start 86.7927 52.5253) (end 86.039 51.7716) (width 0.4) (layer "B.Cu") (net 6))
 (segment (start 83 53) (end 84.25 53) (width 0.4) (layer "B.Cu") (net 6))
 (segment (start 85.7575 65) (end 86.7927 63.9648) (width 0.4) (layer "B.Cu") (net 6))
 (segment (start 83 55.54) (end 85.54 53) (width 0.4) (layer "B.Cu") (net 7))
 (segment (start 83 65) (end 82.7825 65) (width 0.4) (layer "B.Cu") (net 7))
 (segment (start 83 65) (end 83 55.54) (width 0.4) (layer "B.Cu") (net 7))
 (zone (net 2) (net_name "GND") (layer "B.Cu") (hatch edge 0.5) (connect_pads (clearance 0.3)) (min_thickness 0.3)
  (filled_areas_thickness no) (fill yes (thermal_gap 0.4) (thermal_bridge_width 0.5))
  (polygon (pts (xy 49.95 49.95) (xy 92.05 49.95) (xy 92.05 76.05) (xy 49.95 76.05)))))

